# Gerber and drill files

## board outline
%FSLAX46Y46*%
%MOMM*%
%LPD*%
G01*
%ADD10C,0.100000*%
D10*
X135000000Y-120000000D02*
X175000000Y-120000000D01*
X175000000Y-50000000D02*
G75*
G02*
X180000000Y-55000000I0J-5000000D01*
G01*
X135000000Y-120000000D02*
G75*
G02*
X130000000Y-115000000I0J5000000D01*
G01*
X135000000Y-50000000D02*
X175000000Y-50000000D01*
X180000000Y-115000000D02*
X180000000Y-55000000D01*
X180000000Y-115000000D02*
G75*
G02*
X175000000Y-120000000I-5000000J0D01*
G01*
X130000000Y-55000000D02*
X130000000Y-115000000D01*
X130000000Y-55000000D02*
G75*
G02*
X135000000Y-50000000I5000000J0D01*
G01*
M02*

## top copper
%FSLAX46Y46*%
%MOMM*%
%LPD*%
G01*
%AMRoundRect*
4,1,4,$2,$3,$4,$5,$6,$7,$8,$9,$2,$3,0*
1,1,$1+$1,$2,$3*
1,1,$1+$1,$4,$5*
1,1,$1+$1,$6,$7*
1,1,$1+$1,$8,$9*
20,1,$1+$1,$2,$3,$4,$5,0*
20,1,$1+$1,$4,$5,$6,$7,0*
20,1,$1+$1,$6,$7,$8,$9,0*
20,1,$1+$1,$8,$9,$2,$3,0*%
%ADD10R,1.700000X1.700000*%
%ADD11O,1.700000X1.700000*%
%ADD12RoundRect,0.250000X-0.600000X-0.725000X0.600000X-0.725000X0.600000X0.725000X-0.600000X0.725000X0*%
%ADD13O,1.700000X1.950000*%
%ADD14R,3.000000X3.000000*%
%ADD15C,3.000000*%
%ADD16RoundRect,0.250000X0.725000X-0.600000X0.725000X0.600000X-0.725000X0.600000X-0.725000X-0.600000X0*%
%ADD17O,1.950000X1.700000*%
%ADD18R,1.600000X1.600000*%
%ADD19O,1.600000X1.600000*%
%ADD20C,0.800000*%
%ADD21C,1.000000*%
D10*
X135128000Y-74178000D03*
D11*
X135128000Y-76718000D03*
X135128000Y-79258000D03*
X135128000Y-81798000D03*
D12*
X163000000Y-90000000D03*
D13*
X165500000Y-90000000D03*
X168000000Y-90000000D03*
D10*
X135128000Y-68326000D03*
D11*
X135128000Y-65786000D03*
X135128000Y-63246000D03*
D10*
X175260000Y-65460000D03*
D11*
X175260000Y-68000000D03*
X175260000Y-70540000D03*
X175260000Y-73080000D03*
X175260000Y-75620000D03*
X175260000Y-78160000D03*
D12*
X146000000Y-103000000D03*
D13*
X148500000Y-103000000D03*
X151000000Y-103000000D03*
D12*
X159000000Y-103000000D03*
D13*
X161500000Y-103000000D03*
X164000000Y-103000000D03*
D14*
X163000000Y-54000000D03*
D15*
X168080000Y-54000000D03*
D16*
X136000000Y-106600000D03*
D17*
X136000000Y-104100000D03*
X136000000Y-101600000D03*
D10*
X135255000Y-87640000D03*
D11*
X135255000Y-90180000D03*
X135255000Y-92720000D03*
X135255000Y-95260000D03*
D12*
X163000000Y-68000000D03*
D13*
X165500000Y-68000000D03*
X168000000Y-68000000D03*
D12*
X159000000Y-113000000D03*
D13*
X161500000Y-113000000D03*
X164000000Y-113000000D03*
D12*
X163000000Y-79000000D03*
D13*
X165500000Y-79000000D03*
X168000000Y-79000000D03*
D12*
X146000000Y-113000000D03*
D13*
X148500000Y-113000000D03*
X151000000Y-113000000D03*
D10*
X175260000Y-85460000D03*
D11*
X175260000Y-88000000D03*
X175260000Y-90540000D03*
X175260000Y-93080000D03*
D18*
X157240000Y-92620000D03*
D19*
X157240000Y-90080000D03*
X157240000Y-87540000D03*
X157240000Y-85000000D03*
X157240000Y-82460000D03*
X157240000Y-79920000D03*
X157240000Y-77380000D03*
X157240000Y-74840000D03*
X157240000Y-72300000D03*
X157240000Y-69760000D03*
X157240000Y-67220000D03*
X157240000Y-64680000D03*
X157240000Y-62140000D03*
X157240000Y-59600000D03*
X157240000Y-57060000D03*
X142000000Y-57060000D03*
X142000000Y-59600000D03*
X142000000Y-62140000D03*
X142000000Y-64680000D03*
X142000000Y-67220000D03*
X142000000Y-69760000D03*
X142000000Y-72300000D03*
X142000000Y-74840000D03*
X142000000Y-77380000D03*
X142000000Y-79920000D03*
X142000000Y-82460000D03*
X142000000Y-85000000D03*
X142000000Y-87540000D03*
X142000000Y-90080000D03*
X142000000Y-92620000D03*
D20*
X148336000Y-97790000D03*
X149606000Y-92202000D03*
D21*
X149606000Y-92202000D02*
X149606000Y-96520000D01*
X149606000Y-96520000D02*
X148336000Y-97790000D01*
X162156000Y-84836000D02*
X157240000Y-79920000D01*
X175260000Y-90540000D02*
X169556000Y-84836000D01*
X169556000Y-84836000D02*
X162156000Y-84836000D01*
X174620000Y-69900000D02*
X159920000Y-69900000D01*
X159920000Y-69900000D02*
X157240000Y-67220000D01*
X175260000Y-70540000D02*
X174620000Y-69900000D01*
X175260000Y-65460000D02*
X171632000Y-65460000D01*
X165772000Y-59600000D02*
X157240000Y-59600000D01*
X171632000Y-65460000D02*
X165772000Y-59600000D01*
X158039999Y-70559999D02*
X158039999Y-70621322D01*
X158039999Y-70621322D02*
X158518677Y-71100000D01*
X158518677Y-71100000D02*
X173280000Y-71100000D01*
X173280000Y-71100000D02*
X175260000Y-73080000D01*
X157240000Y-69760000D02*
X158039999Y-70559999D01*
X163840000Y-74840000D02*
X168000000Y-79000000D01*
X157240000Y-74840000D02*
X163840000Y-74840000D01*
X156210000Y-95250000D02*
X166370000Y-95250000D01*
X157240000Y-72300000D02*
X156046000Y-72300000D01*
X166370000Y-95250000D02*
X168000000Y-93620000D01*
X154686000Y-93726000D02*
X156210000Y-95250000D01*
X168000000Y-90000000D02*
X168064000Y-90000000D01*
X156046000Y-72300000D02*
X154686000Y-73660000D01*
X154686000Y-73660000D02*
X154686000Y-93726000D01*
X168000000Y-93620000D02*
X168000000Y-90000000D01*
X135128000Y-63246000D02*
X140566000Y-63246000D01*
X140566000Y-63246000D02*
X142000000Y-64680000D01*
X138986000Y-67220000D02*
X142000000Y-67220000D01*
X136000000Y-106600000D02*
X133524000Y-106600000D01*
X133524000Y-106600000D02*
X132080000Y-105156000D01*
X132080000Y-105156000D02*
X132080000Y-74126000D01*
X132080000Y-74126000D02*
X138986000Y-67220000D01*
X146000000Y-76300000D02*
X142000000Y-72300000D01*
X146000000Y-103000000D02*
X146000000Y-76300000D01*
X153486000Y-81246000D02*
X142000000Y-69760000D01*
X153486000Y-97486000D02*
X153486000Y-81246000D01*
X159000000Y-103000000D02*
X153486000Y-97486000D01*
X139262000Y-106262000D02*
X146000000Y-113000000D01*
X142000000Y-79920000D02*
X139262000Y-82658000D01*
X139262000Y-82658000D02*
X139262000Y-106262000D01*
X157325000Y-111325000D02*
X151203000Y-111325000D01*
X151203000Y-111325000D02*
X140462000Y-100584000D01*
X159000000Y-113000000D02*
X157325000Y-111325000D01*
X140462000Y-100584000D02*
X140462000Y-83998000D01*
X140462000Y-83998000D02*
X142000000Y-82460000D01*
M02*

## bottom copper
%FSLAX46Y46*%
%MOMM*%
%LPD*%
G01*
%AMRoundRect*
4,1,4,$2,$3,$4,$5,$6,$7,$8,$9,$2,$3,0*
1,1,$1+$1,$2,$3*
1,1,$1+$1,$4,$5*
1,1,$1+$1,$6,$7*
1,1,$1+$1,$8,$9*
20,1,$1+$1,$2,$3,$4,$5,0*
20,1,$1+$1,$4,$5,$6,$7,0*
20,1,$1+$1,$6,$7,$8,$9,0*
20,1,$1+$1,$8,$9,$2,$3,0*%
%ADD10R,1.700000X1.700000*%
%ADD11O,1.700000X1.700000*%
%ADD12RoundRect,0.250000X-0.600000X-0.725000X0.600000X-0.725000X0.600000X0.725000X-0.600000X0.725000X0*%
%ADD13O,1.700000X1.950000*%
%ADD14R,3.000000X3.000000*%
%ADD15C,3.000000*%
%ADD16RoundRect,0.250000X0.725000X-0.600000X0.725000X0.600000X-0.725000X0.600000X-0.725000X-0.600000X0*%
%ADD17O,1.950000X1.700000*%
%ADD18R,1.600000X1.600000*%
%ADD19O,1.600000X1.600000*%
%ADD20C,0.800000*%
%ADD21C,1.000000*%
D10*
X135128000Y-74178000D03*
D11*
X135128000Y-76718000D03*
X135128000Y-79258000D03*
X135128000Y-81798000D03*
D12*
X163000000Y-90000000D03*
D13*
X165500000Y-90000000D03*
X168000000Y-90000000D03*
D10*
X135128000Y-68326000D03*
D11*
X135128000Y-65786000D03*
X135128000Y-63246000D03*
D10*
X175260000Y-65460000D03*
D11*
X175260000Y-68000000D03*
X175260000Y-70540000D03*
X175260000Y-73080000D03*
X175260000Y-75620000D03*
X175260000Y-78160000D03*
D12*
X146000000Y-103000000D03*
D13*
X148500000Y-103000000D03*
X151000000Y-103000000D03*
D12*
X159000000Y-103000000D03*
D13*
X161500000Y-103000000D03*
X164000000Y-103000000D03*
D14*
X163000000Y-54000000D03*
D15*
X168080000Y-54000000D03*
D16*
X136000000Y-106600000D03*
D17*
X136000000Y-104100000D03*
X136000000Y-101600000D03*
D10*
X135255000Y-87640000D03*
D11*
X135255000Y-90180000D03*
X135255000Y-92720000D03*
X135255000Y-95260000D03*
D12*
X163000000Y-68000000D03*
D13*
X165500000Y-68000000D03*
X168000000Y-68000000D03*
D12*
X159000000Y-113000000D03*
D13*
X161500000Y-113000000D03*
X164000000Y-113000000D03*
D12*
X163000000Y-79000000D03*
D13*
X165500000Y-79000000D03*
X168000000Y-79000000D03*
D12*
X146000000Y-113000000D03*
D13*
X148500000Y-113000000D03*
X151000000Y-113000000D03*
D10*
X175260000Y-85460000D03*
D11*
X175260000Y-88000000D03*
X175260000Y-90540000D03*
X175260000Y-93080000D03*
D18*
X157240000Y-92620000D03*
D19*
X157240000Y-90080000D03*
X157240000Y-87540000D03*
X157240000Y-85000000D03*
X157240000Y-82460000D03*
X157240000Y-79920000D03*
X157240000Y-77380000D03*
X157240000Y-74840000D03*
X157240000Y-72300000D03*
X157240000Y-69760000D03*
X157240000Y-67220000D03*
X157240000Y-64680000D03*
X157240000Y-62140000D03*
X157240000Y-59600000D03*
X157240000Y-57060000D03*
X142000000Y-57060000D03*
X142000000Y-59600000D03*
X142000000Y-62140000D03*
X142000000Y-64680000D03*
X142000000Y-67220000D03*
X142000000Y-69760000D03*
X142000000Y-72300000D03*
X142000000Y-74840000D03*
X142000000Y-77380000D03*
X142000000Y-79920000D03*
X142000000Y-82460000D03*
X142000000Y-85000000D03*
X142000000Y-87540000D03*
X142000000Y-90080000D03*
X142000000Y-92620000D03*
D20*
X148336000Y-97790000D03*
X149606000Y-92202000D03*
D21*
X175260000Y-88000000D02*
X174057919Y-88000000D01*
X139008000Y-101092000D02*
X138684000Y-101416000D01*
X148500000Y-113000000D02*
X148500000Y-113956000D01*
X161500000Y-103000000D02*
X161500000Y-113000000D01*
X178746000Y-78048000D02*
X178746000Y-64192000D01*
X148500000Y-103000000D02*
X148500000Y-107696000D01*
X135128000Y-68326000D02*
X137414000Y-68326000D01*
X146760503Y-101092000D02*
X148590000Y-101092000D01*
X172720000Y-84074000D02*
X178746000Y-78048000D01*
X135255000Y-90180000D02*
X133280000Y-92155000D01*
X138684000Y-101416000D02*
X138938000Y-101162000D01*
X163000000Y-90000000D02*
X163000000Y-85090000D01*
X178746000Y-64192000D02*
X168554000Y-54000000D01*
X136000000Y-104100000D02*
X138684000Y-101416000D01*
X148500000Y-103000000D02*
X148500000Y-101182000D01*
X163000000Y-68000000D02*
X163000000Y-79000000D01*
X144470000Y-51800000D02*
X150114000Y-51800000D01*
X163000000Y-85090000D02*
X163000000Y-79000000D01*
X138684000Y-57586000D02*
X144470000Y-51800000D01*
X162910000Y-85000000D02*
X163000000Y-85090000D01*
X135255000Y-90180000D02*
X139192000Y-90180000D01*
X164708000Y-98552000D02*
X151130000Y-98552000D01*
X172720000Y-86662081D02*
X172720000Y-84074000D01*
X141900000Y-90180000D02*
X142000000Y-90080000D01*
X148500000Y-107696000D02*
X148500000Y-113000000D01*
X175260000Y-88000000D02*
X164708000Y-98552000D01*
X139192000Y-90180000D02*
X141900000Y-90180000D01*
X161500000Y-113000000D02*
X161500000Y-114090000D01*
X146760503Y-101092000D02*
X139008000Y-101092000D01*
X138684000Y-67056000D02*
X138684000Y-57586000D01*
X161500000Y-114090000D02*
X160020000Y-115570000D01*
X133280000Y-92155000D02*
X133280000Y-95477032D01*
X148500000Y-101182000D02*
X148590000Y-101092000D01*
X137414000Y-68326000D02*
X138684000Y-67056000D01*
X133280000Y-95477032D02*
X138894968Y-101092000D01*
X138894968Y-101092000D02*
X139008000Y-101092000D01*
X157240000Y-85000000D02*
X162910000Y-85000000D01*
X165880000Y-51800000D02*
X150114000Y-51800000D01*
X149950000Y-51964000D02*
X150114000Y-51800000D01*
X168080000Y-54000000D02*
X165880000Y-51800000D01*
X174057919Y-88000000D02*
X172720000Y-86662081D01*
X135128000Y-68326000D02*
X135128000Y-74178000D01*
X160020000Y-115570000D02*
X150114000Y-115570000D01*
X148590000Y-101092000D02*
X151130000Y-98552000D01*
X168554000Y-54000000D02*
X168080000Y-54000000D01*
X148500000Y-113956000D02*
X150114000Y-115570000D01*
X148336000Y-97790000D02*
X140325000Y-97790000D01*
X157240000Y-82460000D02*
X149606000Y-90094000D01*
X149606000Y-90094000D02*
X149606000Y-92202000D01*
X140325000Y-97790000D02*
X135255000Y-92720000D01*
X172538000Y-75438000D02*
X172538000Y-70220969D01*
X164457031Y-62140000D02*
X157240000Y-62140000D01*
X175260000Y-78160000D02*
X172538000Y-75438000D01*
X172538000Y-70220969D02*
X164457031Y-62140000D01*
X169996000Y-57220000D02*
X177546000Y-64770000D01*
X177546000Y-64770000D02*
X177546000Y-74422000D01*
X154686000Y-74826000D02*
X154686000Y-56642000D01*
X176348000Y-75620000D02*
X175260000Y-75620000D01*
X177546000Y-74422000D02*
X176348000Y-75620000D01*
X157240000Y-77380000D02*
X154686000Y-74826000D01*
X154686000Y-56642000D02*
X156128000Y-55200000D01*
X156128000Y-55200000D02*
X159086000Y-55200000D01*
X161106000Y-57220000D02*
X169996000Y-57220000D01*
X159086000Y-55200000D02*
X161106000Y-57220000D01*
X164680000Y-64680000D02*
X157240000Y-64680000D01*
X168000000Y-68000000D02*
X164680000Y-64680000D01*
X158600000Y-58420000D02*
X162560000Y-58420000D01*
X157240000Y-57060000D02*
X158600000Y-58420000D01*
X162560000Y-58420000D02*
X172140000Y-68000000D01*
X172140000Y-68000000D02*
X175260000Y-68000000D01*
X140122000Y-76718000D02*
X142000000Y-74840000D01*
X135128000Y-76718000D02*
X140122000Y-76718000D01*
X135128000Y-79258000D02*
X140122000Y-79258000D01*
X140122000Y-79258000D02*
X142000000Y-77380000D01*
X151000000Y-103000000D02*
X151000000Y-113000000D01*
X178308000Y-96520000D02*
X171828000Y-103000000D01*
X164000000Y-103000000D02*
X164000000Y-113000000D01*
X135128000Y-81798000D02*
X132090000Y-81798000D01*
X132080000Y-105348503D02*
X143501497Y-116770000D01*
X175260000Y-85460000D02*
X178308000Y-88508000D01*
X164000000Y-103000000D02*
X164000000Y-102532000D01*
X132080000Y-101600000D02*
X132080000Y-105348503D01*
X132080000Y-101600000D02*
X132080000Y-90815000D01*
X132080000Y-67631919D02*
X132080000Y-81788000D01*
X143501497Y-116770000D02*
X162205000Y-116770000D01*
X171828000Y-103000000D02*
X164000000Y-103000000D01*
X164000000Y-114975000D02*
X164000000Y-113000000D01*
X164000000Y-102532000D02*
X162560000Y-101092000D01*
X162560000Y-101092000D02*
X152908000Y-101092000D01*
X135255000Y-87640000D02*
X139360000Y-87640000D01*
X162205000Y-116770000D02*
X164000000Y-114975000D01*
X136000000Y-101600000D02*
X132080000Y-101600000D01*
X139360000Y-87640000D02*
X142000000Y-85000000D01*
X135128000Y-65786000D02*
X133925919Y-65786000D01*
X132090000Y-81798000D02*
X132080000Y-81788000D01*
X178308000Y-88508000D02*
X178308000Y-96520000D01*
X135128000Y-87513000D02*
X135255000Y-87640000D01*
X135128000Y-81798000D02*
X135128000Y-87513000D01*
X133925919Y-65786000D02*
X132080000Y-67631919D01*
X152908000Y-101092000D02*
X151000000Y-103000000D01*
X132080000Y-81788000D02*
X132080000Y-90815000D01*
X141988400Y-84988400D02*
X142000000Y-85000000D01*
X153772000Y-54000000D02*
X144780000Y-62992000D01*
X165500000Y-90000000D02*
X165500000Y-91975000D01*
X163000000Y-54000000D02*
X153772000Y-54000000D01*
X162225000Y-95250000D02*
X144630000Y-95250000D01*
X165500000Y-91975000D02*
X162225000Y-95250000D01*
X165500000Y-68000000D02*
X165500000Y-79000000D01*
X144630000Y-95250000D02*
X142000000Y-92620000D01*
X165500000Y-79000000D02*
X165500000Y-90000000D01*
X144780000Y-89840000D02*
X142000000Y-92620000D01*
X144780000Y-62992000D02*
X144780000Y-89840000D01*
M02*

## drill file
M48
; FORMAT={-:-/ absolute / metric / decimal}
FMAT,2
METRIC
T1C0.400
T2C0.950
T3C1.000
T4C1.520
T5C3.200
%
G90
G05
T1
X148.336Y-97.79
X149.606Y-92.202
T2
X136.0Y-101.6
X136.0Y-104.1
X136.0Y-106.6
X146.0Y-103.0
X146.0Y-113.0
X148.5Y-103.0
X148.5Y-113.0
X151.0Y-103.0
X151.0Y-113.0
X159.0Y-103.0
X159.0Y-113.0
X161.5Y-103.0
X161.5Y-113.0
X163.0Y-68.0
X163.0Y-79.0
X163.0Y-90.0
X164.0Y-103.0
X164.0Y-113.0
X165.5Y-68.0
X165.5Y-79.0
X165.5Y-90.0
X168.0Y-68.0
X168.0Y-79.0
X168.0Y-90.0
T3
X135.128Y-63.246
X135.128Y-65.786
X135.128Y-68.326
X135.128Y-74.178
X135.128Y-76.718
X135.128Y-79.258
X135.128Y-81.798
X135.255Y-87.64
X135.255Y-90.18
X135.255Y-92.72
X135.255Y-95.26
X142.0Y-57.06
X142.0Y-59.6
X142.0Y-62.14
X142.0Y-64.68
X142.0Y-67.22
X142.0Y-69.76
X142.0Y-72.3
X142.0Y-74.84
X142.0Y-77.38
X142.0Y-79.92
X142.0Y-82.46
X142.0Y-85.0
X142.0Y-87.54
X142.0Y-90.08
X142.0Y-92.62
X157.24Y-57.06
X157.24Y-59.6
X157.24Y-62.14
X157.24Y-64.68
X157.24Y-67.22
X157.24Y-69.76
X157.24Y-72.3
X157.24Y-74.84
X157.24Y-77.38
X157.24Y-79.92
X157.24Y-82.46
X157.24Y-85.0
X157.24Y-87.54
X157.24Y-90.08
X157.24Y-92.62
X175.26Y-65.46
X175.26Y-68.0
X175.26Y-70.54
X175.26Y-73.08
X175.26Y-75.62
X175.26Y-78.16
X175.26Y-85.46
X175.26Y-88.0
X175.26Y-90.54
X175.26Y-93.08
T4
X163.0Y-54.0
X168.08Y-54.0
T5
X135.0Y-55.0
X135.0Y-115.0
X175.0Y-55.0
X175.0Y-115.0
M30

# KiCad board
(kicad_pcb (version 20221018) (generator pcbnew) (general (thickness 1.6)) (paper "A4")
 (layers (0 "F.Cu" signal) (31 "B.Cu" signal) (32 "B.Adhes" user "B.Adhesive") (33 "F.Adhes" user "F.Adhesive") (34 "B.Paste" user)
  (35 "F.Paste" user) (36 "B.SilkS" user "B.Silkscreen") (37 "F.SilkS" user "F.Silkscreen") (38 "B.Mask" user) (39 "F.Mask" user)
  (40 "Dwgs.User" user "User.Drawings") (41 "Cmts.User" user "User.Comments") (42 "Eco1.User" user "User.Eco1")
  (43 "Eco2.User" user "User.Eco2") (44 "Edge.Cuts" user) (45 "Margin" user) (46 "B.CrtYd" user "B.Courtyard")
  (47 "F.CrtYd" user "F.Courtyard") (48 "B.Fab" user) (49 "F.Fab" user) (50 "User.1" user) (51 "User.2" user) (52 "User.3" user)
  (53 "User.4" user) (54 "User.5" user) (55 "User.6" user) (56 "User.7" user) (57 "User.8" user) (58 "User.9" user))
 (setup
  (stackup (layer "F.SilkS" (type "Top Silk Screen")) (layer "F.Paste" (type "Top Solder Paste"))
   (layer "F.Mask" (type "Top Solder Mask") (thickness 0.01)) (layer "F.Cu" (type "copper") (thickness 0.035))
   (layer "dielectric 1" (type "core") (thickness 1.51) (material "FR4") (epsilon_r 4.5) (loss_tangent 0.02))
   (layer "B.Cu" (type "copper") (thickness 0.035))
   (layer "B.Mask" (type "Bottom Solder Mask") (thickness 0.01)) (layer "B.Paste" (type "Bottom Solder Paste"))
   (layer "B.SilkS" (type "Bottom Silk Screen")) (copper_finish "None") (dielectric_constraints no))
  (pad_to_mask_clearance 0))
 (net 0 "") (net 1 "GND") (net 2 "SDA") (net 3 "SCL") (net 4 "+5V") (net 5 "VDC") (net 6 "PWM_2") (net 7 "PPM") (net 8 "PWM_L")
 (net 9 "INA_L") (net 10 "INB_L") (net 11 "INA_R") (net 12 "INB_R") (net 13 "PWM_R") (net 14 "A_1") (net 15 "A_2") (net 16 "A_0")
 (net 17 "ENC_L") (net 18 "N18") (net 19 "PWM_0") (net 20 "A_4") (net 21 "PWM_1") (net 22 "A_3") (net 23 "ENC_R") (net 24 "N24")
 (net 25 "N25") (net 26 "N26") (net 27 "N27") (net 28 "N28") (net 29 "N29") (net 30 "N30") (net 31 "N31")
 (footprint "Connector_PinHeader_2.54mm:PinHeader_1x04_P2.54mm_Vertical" (layer "F.Cu") (at 135.128 74.178)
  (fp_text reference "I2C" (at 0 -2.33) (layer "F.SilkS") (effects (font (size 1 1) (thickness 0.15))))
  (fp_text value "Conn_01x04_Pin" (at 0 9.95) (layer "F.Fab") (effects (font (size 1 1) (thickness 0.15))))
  (pad "1" thru_hole rect (at 0 0) (size 1.7 1.7) (drill 1) (layers "*.Cu" "*.Mask") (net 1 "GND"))
  (pad "2" thru_hole oval (at 0 2.54) (size 1.7 1.7) (drill 1) (layers "*.Cu" "*.Mask") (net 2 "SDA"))
  (pad "3" thru_hole oval (at 0 5.08) (size 1.7 1.7) (drill 1) (layers "*.Cu" "*.Mask") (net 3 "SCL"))
  (pad "4" thru_hole oval (at 0 7.62) (size 1.7 1.7) (drill 1) (layers "*.Cu" "*.Mask") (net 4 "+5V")))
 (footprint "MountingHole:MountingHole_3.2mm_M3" (layer "F.Cu") (at 175 115)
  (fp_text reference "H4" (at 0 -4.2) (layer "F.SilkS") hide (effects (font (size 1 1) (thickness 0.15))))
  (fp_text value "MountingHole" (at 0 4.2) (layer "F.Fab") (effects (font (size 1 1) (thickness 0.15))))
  (pad "" np_thru_hole circle (at 0 0) (size 3.2 3.2) (drill 3.2) (layers "*.Cu" "*.Mask")))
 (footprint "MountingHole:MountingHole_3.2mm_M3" (layer "F.Cu") (at 175 55)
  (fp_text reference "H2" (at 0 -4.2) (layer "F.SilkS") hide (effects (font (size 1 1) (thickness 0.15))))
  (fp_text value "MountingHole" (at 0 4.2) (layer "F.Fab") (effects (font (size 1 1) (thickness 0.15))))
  (pad "" np_thru_hole circle (at 0 0) (size 3.2 3.2) (drill 3.2) (layers "*.Cu" "*.Mask")))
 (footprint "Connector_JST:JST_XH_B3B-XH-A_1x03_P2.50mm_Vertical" (layer "F.Cu") (at 163 90)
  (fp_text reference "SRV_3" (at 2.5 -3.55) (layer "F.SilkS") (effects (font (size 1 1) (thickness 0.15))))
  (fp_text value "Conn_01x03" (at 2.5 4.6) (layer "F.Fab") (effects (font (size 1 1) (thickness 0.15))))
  (pad "1" thru_hole roundrect (at 0 0) (size 1.7 1.95) (drill 0.95) (layers "*.Cu" "*.Mask") (roundrect_rratio 0.147059) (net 1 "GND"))
  (pad "2" thru_hole oval (at 2.5 0) (size 1.7 1.95) (drill 0.95) (layers "*.Cu" "*.Mask") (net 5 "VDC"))
  (pad "3" thru_hole oval (at 5 0) (size 1.7 1.95) (drill 0.95) (layers "*.Cu" "*.Mask") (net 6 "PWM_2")))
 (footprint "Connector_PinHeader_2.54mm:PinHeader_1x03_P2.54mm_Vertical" (layer "F.Cu") (at 135.128 68.326 180)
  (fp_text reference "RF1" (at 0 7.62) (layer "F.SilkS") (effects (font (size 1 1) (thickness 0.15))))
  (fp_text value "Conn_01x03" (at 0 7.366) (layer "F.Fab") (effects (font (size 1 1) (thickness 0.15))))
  (pad "1" thru_hole rect (at 0 0 180) (size 1.7 1.7) (drill 1) (layers "*.Cu" "*.Mask") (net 1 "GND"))
  (pad "2" thru_hole oval (at 0 2.54 180) (size 1.7 1.7) (drill 1) (layers "*.Cu" "*.Mask") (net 4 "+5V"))
  (pad "3" thru_hole oval (at 0 5.08 180) (size 1.7 1.7) (drill 1) (layers "*.Cu" "*.Mask") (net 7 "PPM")))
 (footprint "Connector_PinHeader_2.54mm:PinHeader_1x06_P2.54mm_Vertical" (layer "F.Cu") (at 175.26 65.46)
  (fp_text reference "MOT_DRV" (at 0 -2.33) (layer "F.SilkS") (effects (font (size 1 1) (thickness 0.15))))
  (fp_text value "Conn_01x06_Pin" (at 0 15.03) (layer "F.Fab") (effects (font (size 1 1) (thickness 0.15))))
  (pad "1" thru_hole rect (at 0 0) (size 1.7 1.7) (drill 1) (layers "*.Cu" "*.Mask") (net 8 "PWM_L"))
  (pad "2" thru_hole oval (at 0 2.54) (size 1.7 1.7) (drill 1) (layers "*.Cu" "*.Mask") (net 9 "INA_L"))
  (pad "3" thru_hole oval (at 0 5.08) (size 1.7 1.7) (drill 1) (layers "*.Cu" "*.Mask") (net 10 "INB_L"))
  (pad "4" thru_hole oval (at 0 7.62) (size 1.7 1.7) (drill 1) (layers "*.Cu" "*.Mask") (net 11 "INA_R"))
  (pad "5" thru_hole oval (at 0 10.16) (size 1.7 1.7) (drill 1) (layers "*.Cu" "*.Mask") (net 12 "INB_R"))
  (pad "6" thru_hole oval (at 0 12.7) (size 1.7 1.7) (drill 1) (layers "*.Cu" "*.Mask") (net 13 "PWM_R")))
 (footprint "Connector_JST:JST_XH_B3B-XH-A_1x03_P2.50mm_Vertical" (layer "F.Cu") (at 146 103)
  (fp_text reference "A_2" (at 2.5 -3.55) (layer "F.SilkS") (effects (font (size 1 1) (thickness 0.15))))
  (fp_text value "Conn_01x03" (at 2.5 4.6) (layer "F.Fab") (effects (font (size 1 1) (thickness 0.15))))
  (pad "1" thru_hole roundrect (at 0 0) (size 1.7 1.95) (drill 0.95) (layers "*.Cu" "*.Mask") (roundrect_rratio 0.147059) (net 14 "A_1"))
  (pad "2" thru_hole oval (at 2.5 0) (size 1.7 1.95) (drill 0.95) (layers "*.Cu" "*.Mask") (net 1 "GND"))
  (pad "3" thru_hole oval (at 5 0) (size 1.7 1.95) (drill 0.95) (layers "*.Cu" "*.Mask") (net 4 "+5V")))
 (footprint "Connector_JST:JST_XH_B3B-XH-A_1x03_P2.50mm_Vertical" (layer "F.Cu") (at 159 103)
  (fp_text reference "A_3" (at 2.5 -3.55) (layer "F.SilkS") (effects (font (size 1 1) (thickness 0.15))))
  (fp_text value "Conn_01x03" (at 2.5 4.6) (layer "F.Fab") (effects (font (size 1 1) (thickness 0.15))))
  (pad "1" thru_hole roundrect (at 0 0) (size 1.7 1.95) (drill 0.95) (layers "*.Cu" "*.Mask") (roundrect_rratio 0.147059) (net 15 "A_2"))
  (pad "2" thru_hole oval (at 2.5 0) (size 1.7 1.95) (drill 0.95) (layers "*.Cu" "*.Mask") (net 1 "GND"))
  (pad "3" thru_hole oval (at 5 0) (size 1.7 1.95) (drill 0.95) (layers "*.Cu" "*.Mask") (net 4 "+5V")))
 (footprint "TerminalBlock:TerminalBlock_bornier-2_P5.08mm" (layer "F.Cu") (at 163 54)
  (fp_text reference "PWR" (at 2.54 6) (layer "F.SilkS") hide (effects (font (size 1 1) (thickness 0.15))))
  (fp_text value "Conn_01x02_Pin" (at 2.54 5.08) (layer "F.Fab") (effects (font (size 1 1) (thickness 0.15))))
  (pad "1" thru_hole rect (at 0 0) (size 3 3) (drill 1.52) (layers "*.Cu" "*.Mask") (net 5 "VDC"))
  (pad "2" thru_hole circle (at 5.08 0) (size 3 3) (drill 1.52) (layers "*.Cu" "*.Mask") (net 1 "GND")))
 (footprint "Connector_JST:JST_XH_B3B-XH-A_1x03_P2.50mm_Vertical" (layer "F.Cu") (at 136 106.6 90)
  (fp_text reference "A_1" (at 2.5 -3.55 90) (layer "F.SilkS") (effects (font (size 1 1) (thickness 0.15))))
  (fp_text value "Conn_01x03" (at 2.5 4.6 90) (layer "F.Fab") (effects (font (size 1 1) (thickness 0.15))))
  (pad "1" thru_hole roundrect (at 0 0 90) (size 1.7 1.95) (drill 0.95) (layers "*.Cu" "*.Mask") (roundrect_rratio 0.147059) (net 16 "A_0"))
  (pad "2" thru_hole oval (at 2.5 0 90) (size 1.7 1.95) (drill 0.95) (layers "*.Cu" "*.Mask") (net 1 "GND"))
  (pad "3" thru_hole oval (at 5 0 90) (size 1.7 1.95) (drill 0.95) (layers "*.Cu" "*.Mask") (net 4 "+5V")))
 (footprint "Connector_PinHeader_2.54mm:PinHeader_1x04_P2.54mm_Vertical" (layer "F.Cu") (at 135.255 87.64)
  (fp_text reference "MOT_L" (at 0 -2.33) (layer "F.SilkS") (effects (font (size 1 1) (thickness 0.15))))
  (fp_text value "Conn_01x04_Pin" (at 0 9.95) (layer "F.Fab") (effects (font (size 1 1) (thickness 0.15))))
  (pad "1" thru_hole rect (at 0 0) (size 1.7 1.7) (drill 1) (layers "*.Cu" "*.Mask") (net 4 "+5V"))
  (pad "2" thru_hole oval (at 0 2.54) (size 1.7 1.7) (drill 1) (layers "*.Cu" "*.Mask") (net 1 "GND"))
  (pad "3" thru_hole oval (at 0 5.08) (size 1.7 1.7) (drill 1) (layers "*.Cu" "*.Mask") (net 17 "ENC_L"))
  (pad "4" thru_hole oval (at 0 7.62) (size 1.7 1.7) (drill 1) (layers "*.Cu" "*.Mask") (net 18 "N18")))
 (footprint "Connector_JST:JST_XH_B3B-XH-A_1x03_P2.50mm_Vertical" (layer "F.Cu") (at 163 68)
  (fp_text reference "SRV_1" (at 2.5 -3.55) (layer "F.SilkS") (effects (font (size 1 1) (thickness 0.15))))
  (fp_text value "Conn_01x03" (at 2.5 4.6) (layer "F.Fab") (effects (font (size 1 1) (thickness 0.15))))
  (pad "1" thru_hole roundrect (at 0 0) (size 1.7 1.95) (drill 0.95) (layers "*.Cu" "*.Mask") (roundrect_rratio 0.147059) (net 1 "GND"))
  (pad "2" thru_hole oval (at 2.5 0) (size 1.7 1.95) (drill 0.95) (layers "*.Cu" "*.Mask") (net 5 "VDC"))
  (pad "3" thru_hole oval (at 5 0) (size 1.7 1.95) (drill 0.95) (layers "*.Cu" "*.Mask") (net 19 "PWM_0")))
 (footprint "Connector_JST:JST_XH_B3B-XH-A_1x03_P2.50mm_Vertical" (layer "F.Cu") (at 159 113)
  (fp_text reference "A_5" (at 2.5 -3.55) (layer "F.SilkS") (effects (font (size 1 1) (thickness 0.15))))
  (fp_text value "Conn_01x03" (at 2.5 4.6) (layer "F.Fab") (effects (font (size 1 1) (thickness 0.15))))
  (pad "1" thru_hole roundrect (at 0 0) (size 1.7 1.95) (drill 0.95) (layers "*.Cu" "*.Mask") (roundrect_rratio 0.147059) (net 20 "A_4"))
  (pad "2" thru_hole oval (at 2.5 0) (size 1.7 1.95) (drill 0.95) (layers "*.Cu" "*.Mask") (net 1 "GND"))
  (pad "3" thru_hole oval (at 5 0) (size 1.7 1.95) (drill 0.95) (layers "*.Cu" "*.Mask") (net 4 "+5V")))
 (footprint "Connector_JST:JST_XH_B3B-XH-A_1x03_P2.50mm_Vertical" (layer "F.Cu") (at 163 79)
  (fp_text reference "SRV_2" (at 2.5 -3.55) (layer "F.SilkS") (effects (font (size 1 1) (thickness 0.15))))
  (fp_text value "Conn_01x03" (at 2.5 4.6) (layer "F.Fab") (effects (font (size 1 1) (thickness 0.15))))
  (pad "1" thru_hole roundrect (at 0 0) (size 1.7 1.95) (drill 0.95) (layers "*.Cu" "*.Mask") (roundrect_rratio 0.147059) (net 1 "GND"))
  (pad "2" thru_hole oval (at 2.5 0) (size 1.7 1.95) (drill 0.95) (layers "*.Cu" "*.Mask") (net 5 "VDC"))
  (pad "3" thru_hole oval (at 5 0) (size 1.7 1.95) (drill 0.95) (layers "*.Cu" "*.Mask") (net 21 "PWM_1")))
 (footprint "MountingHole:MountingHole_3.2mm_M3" (layer "F.Cu") (at 135 115)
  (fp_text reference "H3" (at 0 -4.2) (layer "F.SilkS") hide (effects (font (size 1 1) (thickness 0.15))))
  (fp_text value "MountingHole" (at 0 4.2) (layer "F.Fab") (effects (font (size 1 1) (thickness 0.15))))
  (pad "" np_thru_hole circle (at 0 0) (size 3.2 3.2) (drill 3.2) (layers "*.Cu" "*.Mask")))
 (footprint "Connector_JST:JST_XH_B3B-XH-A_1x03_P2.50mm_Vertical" (layer "F.Cu") (at 146 113)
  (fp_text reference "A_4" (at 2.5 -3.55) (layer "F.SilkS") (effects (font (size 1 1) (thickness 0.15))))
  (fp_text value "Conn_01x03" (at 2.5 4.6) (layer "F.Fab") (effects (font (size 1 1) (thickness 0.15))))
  (pad "1" thru_hole roundrect (at 0 0) (size 1.7 1.95) (drill 0.95) (layers "*.Cu" "*.Mask") (roundrect_rratio 0.147059) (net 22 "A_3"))
  (pad "2" thru_hole oval (at 2.5 0) (size 1.7 1.95) (drill 0.95) (layers "*.Cu" "*.Mask") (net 1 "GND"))
  (pad "3" thru_hole oval (at 5 0) (size 1.7 1.95) (drill 0.95) (layers "*.Cu" "*.Mask") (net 4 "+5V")))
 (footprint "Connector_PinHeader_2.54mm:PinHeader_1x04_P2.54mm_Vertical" (layer "F.Cu") (at 175.26 85.46)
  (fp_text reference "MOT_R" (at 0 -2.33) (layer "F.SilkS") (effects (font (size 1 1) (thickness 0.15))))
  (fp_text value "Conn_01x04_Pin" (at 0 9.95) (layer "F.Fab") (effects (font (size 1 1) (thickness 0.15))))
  (pad "1" thru_hole rect (at 0 0) (size 1.7 1.7) (drill 1) (layers "*.Cu" "*.Mask") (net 4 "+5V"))
  (pad "2" thru_hole oval (at 0 2.54) (size 1.7 1.7) (drill 1) (layers "*.Cu" "*.Mask") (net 1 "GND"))
  (pad "3" thru_hole oval (at 0 5.08) (size 1.7 1.7) (drill 1) (layers "*.Cu" "*.Mask") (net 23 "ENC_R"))
  (pad "4" thru_hole oval (at 0 7.62) (size 1.7 1.7) (drill 1) (layers "*.Cu" "*.Mask") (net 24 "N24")))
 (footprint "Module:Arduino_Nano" (layer "F.Cu") (at 157.24 92.62 180)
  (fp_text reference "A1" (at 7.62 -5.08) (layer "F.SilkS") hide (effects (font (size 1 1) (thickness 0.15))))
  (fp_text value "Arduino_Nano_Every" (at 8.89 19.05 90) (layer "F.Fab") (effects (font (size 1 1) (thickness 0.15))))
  (pad "1" thru_hole rect (at 0 0 180) (size 1.6 1.6) (drill 1) (layers "*.Cu" "*.Mask") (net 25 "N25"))
  (pad "2" thru_hole oval (at 0 2.54 180) (size 1.6 1.6) (drill 1) (layers "*.Cu" "*.Mask") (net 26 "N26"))
  (pad "3" thru_hole oval (at 0 5.08 180) (size 1.6 1.6) (drill 1) (layers "*.Cu" "*.Mask") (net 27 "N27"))
  (pad "4" thru_hole oval (at 0 7.62 180) (size 1.6 1.6) (drill 1) (layers "*.Cu" "*.Mask") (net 1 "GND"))
  (pad "5" thru_hole oval (at 0 10.16 180) (size 1.6 1.6) (drill 1) (layers "*.Cu" "*.Mask") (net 17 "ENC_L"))
  (pad "6" thru_hole oval (at 0 12.7 180) (size 1.6 1.6) (drill 1) (layers "*.Cu" "*.Mask") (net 23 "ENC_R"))
  (pad "7" thru_hole oval (at 0 15.24 180) (size 1.6 1.6) (drill 1) (layers "*.Cu" "*.Mask") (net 12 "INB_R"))
  (pad "8" thru_hole oval (at 0 17.78 180) (size 1.6 1.6) (drill 1) (layers "*.Cu" "*.Mask") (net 21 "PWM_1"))
  (pad "9" thru_hole oval (at 0 20.32 180) (size 1.6 1.6) (drill 1) (layers "*.Cu" "*.Mask") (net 6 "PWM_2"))
  (pad "10" thru_hole oval (at 0 22.86 180) (size 1.6 1.6) (drill 1) (layers "*.Cu" "*.Mask") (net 11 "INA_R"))
  (pad "11" thru_hole oval (at 0 25.4 180) (size 1.6 1.6) (drill 1) (layers "*.Cu" "*.Mask") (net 10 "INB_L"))
  (pad "12" thru_hole oval (at 0 27.94 180) (size 1.6 1.6) (drill 1) (layers "*.Cu" "*.Mask") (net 19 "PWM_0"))
  (pad "13" thru_hole oval (at 0 30.48 180) (size 1.6 1.6) (drill 1) (layers "*.Cu" "*.Mask") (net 13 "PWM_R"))
  (pad "14" thru_hole oval (at 0 33.02 180) (size 1.6 1.6) (drill 1) (layers "*.Cu" "*.Mask") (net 8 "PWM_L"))
  (pad "15" thru_hole oval (at 0 35.56 180) (size 1.6 1.6) (drill 1) (layers "*.Cu" "*.Mask") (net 9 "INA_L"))
  (pad "16" thru_hole oval (at 15.24 35.56 180) (size 1.6 1.6) (drill 1) (layers "*.Cu" "*.Mask") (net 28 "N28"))
  (pad "17" thru_hole oval (at 15.24 33.02 180) (size 1.6 1.6) (drill 1) (layers "*.Cu" "*.Mask") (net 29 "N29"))
  (pad "18" thru_hole oval (at 15.24 30.48 180) (size 1.6 1.6) (drill 1) (layers "*.Cu" "*.Mask") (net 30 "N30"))
  (pad "19" thru_hole oval (at 15.24 27.94 180) (size 1.6 1.6) (drill 1) (layers "*.Cu" "*.Mask") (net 7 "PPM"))
  (pad "20" thru_hole oval (at 15.24 25.4 180) (size 1.6 1.6) (drill 1) (layers "*.Cu" "*.Mask") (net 16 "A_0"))
  (pad "21" thru_hole oval (at 15.24 22.86 180) (size 1.6 1.6) (drill 1) (layers "*.Cu" "*.Mask") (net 15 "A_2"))
  (pad "22" thru_hole oval (at 15.24 20.32 180) (size 1.6 1.6) (drill 1) (layers "*.Cu" "*.Mask") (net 14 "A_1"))
  (pad "23" thru_hole oval (at 15.24 17.78 180) (size 1.6 1.6) (drill 1) (layers "*.Cu" "*.Mask") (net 2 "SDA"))
  (pad "24" thru_hole oval (at 15.24 15.24 180) (size 1.6 1.6) (drill 1) (layers "*.Cu" "*.Mask") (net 3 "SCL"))
  (pad "25" thru_hole oval (at 15.24 12.7 180) (size 1.6 1.6) (drill 1) (layers "*.Cu" "*.Mask") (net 22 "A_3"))
  (pad "26" thru_hole oval (at 15.24 10.16 180) (size 1.6 1.6) (drill 1) (layers "*.Cu" "*.Mask") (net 20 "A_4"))
  (pad "27" thru_hole oval (at 15.24 7.62 180) (size 1.6 1.6) (drill 1) (layers "*.Cu" "*.Mask") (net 4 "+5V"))
  (pad "28" thru_hole oval (at 15.24 5.08 180) (size 1.6 1.6) (drill 1) (layers "*.Cu" "*.Mask") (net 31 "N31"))
  (pad "29" thru_hole oval (at 15.24 2.54 180) (size 1.6 1.6) (drill 1) (layers "*.Cu" "*.Mask") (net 1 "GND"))
  (pad "30" thru_hole oval (at 15.24 0 180) (size 1.6 1.6) (drill 1) (layers "*.Cu" "*.Mask") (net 5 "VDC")))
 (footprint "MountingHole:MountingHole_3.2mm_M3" (layer "F.Cu") (at 135 55)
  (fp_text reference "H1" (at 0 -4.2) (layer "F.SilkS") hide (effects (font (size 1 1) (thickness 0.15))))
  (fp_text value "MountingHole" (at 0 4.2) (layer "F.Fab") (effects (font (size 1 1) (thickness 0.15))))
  (pad "" np_thru_hole circle (at 0 0) (size 3.2 3.2) (drill 3.2) (layers "*.Cu" "*.Mask")))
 (gr_line (start 135 120) (end 175 120) (stroke (width 0.1) (type default)) (layer "Edge.Cuts"))
 (gr_arc (start 175 50) (mid 178.535534 51.464466) (end 180 55) (stroke (width 0.1) (type default)) (layer "Edge.Cuts"))
 (gr_arc (start 135 120) (mid 131.464466 118.535534) (end 130 115) (stroke (width 0.1) (type default)) (layer "Edge.Cuts"))
 (gr_line (start 135 50) (end 175 50) (stroke (width 0.1) (type default)) (layer "Edge.Cuts"))
 (gr_line (start 180 115) (end 180 55) (stroke (width 0.1) (type default)) (layer "Edge.Cuts"))
 (gr_arc (start 180 115) (mid 178.535534 118.535534) (end 175 120) (stroke (width 0.1) (type default)) (layer "Edge.Cuts"))
 (gr_line (start 130 55) (end 130 115) (stroke (width 0.1) (type default)) (layer "Edge.Cuts"))
 (gr_arc (start 130 55) (mid 131.464466 51.464466) (end 135 50) (stroke (width 0.1) (type default)) (layer "Edge.Cuts"))
 (segment (start 175.26 88) (end 174.057919 88) (width 1) (layer "B.Cu") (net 1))
 (segment (start 139.008 101.092) (end 138.684 101.416) (width 1) (layer "B.Cu") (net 1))
 (segment (start 148.5 113) (end 148.5 113.956) (width 1) (layer "B.Cu") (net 1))
 (segment (start 161.5 103) (end 161.5 113) (width 1) (layer "B.Cu") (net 1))
 (segment (start 178.746 78.048) (end 178.746 64.192) (width 1) (layer "B.Cu") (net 1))
 (segment (start 148.5 103) (end 148.5 107.696) (width 1) (layer "B.Cu") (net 1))
 (segment (start 135.128 68.326) (end 137.414 68.326) (width 1) (layer "B.Cu") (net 1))
 (segment (start 146.760503 101.092) (end 148.59 101.092) (width 1) (layer "B.Cu") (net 1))
 (segment (start 172.72 84.074) (end 178.746 78.048) (width 1) (layer "B.Cu") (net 1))
 (segment (start 135.255 90.18) (end 133.28 92.155) (width 1) (layer "B.Cu") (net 1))
 (segment (start 138.684 101.416) (end 138.938 101.162) (width 1) (layer "B.Cu") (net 1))
 (segment (start 163 90) (end 163 85.09) (width 1) (layer "B.Cu") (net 1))
 (segment (start 178.746 64.192) (end 168.554 54) (width 1) (layer "B.Cu") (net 1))
 (segment (start 136 104.1) (end 138.684 101.416) (width 1) (layer "B.Cu") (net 1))
 (segment (start 148.5 103) (end 148.5 101.182) (width 1) (layer "B.Cu") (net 1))
 (segment (start 163 68) (end 163 79) (width 1) (layer "B.Cu") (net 1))
 (segment (start 144.47 51.8) (end 150.114 51.8) (width 1) (layer "B.Cu") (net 1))
 (segment (start 163 85.09) (end 163 79) (width 1) (layer "B.Cu") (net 1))
 (segment (start 138.684 57.586) (end 144.47 51.8) (width 1) (layer "B.Cu") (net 1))
 (segment (start 162.91 85) (end 163 85.09) (width 1) (layer "B.Cu") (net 1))
 (segment (start 135.255 90.18) (end 139.192 90.18) (width 1) (layer "B.Cu") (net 1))
 (segment (start 164.708 98.552) (end 151.13 98.552) (width 1) (layer "B.Cu") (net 1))
 (segment (start 172.72 86.662081) (end 172.72 84.074) (width 1) (layer "B.Cu") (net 1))
 (segment (start 141.9 90.18) (end 142 90.08) (width 1) (layer "B.Cu") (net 1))
 (segment (start 148.5 107.696) (end 148.5 113) (width 1) (layer "B.Cu") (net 1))
 (segment (start 175.26 88) (end 164.708 98.552) (width 1) (layer "B.Cu") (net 1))
 (segment (start 139.192 90.18) (end 141.9 90.18) (width 1) (layer "B.Cu") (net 1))
 (segment (start 161.5 113) (end 161.5 114.09) (width 1) (layer "B.Cu") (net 1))
 (segment (start 146.760503 101.092) (end 139.008 101.092) (width 1) (layer "B.Cu") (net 1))
 (segment (start 138.684 67.056) (end 138.684 57.586) (width 1) (layer "B.Cu") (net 1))
 (segment (start 161.5 114.09) (end 160.02 115.57) (width 1) (layer "B.Cu") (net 1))
 (segment (start 133.28 92.155) (end 133.28 95.477032) (width 1) (layer "B.Cu") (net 1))
 (segment (start 148.5 101.182) (end 148.59 101.092) (width 1) (layer "B.Cu") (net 1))
 (segment (start 137.414 68.326) (end 138.684 67.056) (width 1) (layer "B.Cu") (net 1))
 (segment (start 133.28 95.477032) (end 138.894968 101.092) (width 1) (layer "B.Cu") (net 1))
 (segment (start 138.894968 101.092) (end 139.008 101.092) (width 1) (layer "B.Cu") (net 1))
 (segment (start 157.24 85) (end 162.91 85) (width 1) (layer "B.Cu") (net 1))
 (segment (start 165.88 51.8) (end 150.114 51.8) (width 1) (layer "B.Cu") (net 1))
 (segment (start 149.95 51.964) (end 150.114 51.8) (width 1) (layer "B.Cu") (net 1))
 (segment (start 168.08 54) (end 165.88 51.8) (width 1) (layer "B.Cu") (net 1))
 (segment (start 174.057919 88) (end 172.72 86.662081) (width 1) (layer "B.Cu") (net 1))
 (segment (start 135.128 68.326) (end 135.128 74.178) (width 1) (layer "B.Cu") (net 1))
 (segment (start 160.02 115.57) (end 150.114 115.57) (width 1) (layer "B.Cu") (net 1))
 (segment (start 148.59 101.092) (end 151.13 98.552) (width 1) (layer "B.Cu") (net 1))
 (segment (start 168.554 54) (end 168.08 54) (width 1) (layer "B.Cu") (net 1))
 (segment (start 148.5 113.956) (end 150.114 115.57) (width 1) (layer "B.Cu") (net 1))
 (segment (start 149.606 92.202) (end 149.606 96.52) (width 1) (layer "F.Cu") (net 17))
 (segment (start 149.606 96.52) (end 148.336 97.79) (width 1) (layer "F.Cu") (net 17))
 (via (at 148.336 97.79) (size 0.8) (drill 0.4) (layers "F.Cu" "B.Cu") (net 17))
 (via (at 149.606 92.202) (size 0.8) (drill 0.4) (layers "F.Cu" "B.Cu") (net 17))
 (segment (start 148.336 97.79) (end 140.325 97.79) (width 1) (layer "B.Cu") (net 17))
 (segment (start 157.24 82.46) (end 149.606 90.094) (width 1) (layer "B.Cu") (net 17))
 (segment (start 149.606 90.094) (end 149.606 92.202) (width 1) (layer "B.Cu") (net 17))
 (segment (start 140.325 97.79) (end 135.255 92.72) (width 1) (layer "B.Cu") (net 17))
 (segment (start 162.156 84.836) (end 157.24 79.92) (width 1) (layer "F.Cu") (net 23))
 (segment (start 175.26 90.54) (end 169.556 84.836) (width 1) (layer "F.Cu") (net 23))
 (segment (start 169.556 84.836) (end 162.156 84.836) (width 1) (layer "F.Cu") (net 23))
 (segment (start 174.62 69.9) (end 159.92 69.9) (width 1) (layer "F.Cu") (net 10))
 (segment (start 159.92 69.9) (end 157.24 67.22) (width 1) (layer "F.Cu") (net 10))
 (segment (start 175.26 70.54) (end 174.62 69.9) (width 1) (layer "F.Cu") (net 10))
 (segment (start 175.26 65.46) (end 171.632 65.46) (width 1) (layer "F.Cu") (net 8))
 (segment (start 165.772 59.6) (end 157.24 59.6) (width 1) (layer "F.Cu") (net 8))
 (segment (start 171.632 65.46) (end 165.772 59.6) (width 1) (layer "F.Cu") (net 8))
 (segment (start 172.538 75.438) (end 172.538 70.220969) (width 1) (layer "B.Cu") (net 13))
 (segment (start 164.457031 62.14) (end 157.24 62.14) (width 1) (layer "B.Cu") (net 13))
 (segment (start 175.26 78.16) (end 172.538 75.438) (width 1) (layer "B.Cu") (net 13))
 (segment (start 172.538 70.220969) (end 164.457031 62.14) (width 1) (layer "B.Cu") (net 13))
 (segment (start 169.996 57.22) (end 177.546 64.77) (width 1) (layer "B.Cu") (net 12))
 (segment (start 177.546 64.77) (end 177.546 74.422) (width 1) (layer "B.Cu") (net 12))
 (segment (start 154.686 74.826) (end 154.686 56.642) (width 1) (layer "B.Cu") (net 12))
 (segment (start 176.348 75.62) (end 175.26 75.62) (width 1) (layer "B.Cu") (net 12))
 (segment (start 177.546 74.422) (end 176.348 75.62) (width 1) (layer "B.Cu") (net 12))
 (segment (start 157.24 77.38) (end 154.686 74.826) (width 1) (layer "B.Cu") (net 12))
 (segment (start 154.686 56.642) (end 156.128 55.2) (width 1) (layer "B.Cu") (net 12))
 (segment (start 156.128 55.2) (end 159.086 55.2) (width 1) (layer "B.Cu") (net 12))
 (segment (start 161.106 57.22) (end 169.996 57.22) (width 1) (layer "B.Cu") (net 12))
 (segment (start 159.086 55.2) (end 161.106 57.22) (width 1) (layer "B.Cu") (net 12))
 (segment (start 158.039999 70.559999) (end 158.039999 70.621322) (width 1) (layer "F.Cu") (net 11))
 (segment (start 158.039999 70.621322) (end 158.518677 71.1) (width 1) (layer "F.Cu") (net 11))
 (segment (start 158.518677 71.1) (end 173.28 71.1) (width 1) (layer "F.Cu") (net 11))
 (segment (start 173.28 71.1) (end 175.26 73.08) (width 1) (layer "F.Cu") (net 11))
 (segment (start 157.24 69.76) (end 158.039999 70.559999) (width 1) (layer "F.Cu") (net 11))
 (segment (start 164.68 64.68) (end 157.24 64.68) (width 1) (layer "B.Cu") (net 19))
 (segment (start 168 68) (end 164.68 64.68) (width 1) (layer "B.Cu") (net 19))
 (segment (start 163.84 74.84) (end 168 79) (width 1) (layer "F.Cu") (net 21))
 (segment (start 157.24 74.84) (end 163.84 74.84) (width 1) (layer "F.Cu") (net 21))
 (segment (start 156.21 95.25) (end 166.37 95.25) (width 1) (layer "F.Cu") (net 6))
 (segment (start 157.24 72.3) (end 156.046 72.3) (width 1) (layer "F.Cu") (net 6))
 (segment (start 166.37 95.25) (end 168 93.62) (width 1) (layer "F.Cu") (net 6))
 (segment (start 154.686 93.726) (end 156.21 95.25) (width 1) (layer "F.Cu") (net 6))
 (segment (start 168 90) (end 168.064 90) (width 1) (layer "F.Cu") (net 6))
 (segment (start 156.046 72.3) (end 154.686 73.66) (width 1) (layer "F.Cu") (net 6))
 (segment (start 154.686 73.66) (end 154.686 93.726) (width 1) (layer "F.Cu") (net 6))
 (segment (start 168 93.62) (end 168 90) (width 1) (layer "F.Cu") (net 6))
 (segment (start 158.6 58.42) (end 162.56 58.42) (width 1) (layer "B.Cu") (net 9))
 (segment (start 157.24 57.06) (end 158.6 58.42) (width 1) (layer "B.Cu") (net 9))
 (segment (start 162.56 58.42) (end 172.14 68) (width 1) (layer "B.Cu") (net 9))
 (segment (start 172.14 68) (end 175.26 68) (width 1) (layer "B.Cu") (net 9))
 (segment (start 135.128 63.246) (end 140.566 63.246) (width 1) (layer "F.Cu") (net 7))
 (segment (start 140.566 63.246) (end 142 64.68) (width 1) (layer "F.Cu") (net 7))
 (segment (start 138.986 67.22) (end 142 67.22) (width 1) (layer "F.Cu") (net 16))
 (segment (start 136 106.6) (end 133.524 106.6) (width 1) (layer "F.Cu") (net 16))
 (segment (start 133.524 106.6) (end 132.08 105.156) (width 1) (layer "F.Cu") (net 16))
 (segment (start 132.08 105.156) (end 132.08 74.126) (width 1) (layer "F.Cu") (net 16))
 (segment (start 132.08 74.126) (end 138.986 67.22) (width 1) (layer "F.Cu") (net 16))
 (segment (start 146 76.3) (end 142 72.3) (width 1) (layer "F.Cu") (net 14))
 (segment (start 146 103) (end 146 76.3) (width 1) (layer "F.Cu") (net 14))
 (segment (start 153.486 81.246) (end 142 69.76) (width 1) (layer "F.Cu") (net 15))
 (segment (start 153.486 97.486) (end 153.486 81.246) (width 1) (layer "F.Cu") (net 15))
 (segment (start 159 103) (end 153.486 97.486) (width 1) (layer "F.Cu") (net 15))
 (segment (start 140.122 76.718) (end 142 74.84) (width 1) (layer "B.Cu") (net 2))
 (segment (start 135.128 76.718) (end 140.122 76.718) (width 1) (layer "B.Cu") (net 2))
 (segment (start 135.128 79.258) (end 140.122 79.258) (width 1) (layer "B.Cu") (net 3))
 (segment (start 140.122 79.258) (end 142 77.38) (width 1) (layer "B.Cu") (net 3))
 (segment (start 139.262 106.262) (end 146 113) (width 1) (layer "F.Cu") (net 22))
 (segment (start 142 79.92) (end 139.262 82.658) (width 1) (layer "F.Cu") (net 22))
 (segment (start 139.262 82.658) (end 139.262 106.262) (width 1) (layer "F.Cu") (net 22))
 (segment (start 157.325 111.325) (end 151.203 111.325) (width 1) (layer "F.Cu") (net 20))
 (segment (start 151.203 111.325) (end 140.462 100.584) (width 1) (layer "F.Cu") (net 20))
 (segment (start 159 113) (end 157.325 111.325) (width 1) (layer "F.Cu") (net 20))
 (segment (start 140.462 100.584) (end 140.462 83.998) (width 1) (layer "F.Cu") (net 20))
 (segment (start 140.462 83.998) (end 142 82.46) (width 1) (layer "F.Cu") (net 20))
 (segment (start 151 103) (end 151 113) (width 1) (layer "B.Cu") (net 4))
 (segment (start 178.308 96.52) (end 171.828 103) (width 1) (layer "B.Cu") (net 4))
 (segment (start 164 103) (end 164 113) (width 1) (layer "B.Cu") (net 4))
 (segment (start 135.128 81.798) (end 132.09 81.798) (width 1) (layer "B.Cu") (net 4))
 (segment (start 132.08 105.348503) (end 143.501497 116.77) (width 1) (layer "B.Cu") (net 4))
 (segment (start 175.26 85.46) (end 178.308 88.508) (width 1) (layer "B.Cu") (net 4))
 (segment (start 164 103) (end 164 102.532) (width 1) (layer "B.Cu") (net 4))
 (segment (start 132.08 101.6) (end 132.08 105.348503) (width 1) (layer "B.Cu") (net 4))
 (segment (start 132.08 101.6) (end 132.08 90.815) (width 1) (layer "B.Cu") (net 4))
 (segment (start 132.08 67.631919) (end 132.08 81.788) (width 1) (layer "B.Cu") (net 4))
 (segment (start 143.501497 116.77) (end 162.205 116.77) (width 1) (layer "B.Cu") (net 4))
 (segment (start 171.828 103) (end 164 103) (width 1) (layer "B.Cu") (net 4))
 (segment (start 164 114.975) (end 164 113) (width 1) (layer "B.Cu") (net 4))
 (segment (start 164 102.532) (end 162.56 101.092) (width 1) (layer "B.Cu") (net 4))
 (segment (start 162.56 101.092) (end 152.908 101.092) (width 1) (layer "B.Cu") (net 4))
 (segment (start 135.255 87.64) (end 139.36 87.64) (width 1) (layer "B.Cu") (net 4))
 (segment (start 162.205 116.77) (end 164 114.975) (width 1) (layer "B.Cu") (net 4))
 (segment (start 136 101.6) (end 132.08 101.6) (width 1) (layer "B.Cu") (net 4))
 (segment (start 139.36 87.64) (end 142 85) (width 1) (layer "B.Cu") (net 4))
 (segment (start 135.128 65.786) (end 133.925919 65.786) (width 1) (layer "B.Cu") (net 4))
 (segment (start 132.09 81.798) (end 132.08 81.788) (width 1) (layer "B.Cu") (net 4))
 (segment (start 178.308 88.508) (end 178.308 96.52) (width 1) (layer "B.Cu") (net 4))
 (segment (start 135.128 87.513) (end 135.255 87.64) (width 1) (layer "B.Cu") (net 4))
 (segment (start 135.128 81.798) (end 135.128 87.513) (width 1) (layer "B.Cu") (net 4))
 (segment (start 133.925919 65.786) (end 132.08 67.631919) (width 1) (layer "B.Cu") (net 4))
 (segment (start 152.908 101.092) (end 151 103) (width 1) (layer "B.Cu") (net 4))
 (segment (start 132.08 81.788) (end 132.08 90.815) (width 1) (layer "B.Cu") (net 4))
 (segment (start 141.9884 84.9884) (end 142 85) (width 1) (layer "B.Cu") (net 4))
 (segment (start 153.772 54) (end 144.78 62.992) (width 1) (layer "B.Cu") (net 5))
 (segment (start 165.5 90) (end 165.5 91.975) (width 1) (layer "B.Cu") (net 5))
 (segment (start 163 54) (end 153.772 54) (width 1) (layer "B.Cu") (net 5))
 (segment (start 162.225 95.25) (end 144.63 95.25) (width 1) (layer "B.Cu") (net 5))
 (segment (start 165.5 91.975) (end 162.225 95.25) (width 1) (layer "B.Cu") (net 5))
 (segment (start 165.5 68) (end 165.5 79) (width 1) (layer "B.Cu") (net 5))
 (segment (start 144.63 95.25) (end 142 92.62) (width 1) (layer "B.Cu") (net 5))
 (segment (start 165.5 79) (end 165.5 90) (width 1) (layer "B.Cu") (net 5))
 (segment (start 144.78 89.84) (end 142 92.62) (width 1) (layer "B.Cu") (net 5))
 (segment (start 144.78 62.992) (end 144.78 89.84) (width 1) (layer "B.Cu") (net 5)))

